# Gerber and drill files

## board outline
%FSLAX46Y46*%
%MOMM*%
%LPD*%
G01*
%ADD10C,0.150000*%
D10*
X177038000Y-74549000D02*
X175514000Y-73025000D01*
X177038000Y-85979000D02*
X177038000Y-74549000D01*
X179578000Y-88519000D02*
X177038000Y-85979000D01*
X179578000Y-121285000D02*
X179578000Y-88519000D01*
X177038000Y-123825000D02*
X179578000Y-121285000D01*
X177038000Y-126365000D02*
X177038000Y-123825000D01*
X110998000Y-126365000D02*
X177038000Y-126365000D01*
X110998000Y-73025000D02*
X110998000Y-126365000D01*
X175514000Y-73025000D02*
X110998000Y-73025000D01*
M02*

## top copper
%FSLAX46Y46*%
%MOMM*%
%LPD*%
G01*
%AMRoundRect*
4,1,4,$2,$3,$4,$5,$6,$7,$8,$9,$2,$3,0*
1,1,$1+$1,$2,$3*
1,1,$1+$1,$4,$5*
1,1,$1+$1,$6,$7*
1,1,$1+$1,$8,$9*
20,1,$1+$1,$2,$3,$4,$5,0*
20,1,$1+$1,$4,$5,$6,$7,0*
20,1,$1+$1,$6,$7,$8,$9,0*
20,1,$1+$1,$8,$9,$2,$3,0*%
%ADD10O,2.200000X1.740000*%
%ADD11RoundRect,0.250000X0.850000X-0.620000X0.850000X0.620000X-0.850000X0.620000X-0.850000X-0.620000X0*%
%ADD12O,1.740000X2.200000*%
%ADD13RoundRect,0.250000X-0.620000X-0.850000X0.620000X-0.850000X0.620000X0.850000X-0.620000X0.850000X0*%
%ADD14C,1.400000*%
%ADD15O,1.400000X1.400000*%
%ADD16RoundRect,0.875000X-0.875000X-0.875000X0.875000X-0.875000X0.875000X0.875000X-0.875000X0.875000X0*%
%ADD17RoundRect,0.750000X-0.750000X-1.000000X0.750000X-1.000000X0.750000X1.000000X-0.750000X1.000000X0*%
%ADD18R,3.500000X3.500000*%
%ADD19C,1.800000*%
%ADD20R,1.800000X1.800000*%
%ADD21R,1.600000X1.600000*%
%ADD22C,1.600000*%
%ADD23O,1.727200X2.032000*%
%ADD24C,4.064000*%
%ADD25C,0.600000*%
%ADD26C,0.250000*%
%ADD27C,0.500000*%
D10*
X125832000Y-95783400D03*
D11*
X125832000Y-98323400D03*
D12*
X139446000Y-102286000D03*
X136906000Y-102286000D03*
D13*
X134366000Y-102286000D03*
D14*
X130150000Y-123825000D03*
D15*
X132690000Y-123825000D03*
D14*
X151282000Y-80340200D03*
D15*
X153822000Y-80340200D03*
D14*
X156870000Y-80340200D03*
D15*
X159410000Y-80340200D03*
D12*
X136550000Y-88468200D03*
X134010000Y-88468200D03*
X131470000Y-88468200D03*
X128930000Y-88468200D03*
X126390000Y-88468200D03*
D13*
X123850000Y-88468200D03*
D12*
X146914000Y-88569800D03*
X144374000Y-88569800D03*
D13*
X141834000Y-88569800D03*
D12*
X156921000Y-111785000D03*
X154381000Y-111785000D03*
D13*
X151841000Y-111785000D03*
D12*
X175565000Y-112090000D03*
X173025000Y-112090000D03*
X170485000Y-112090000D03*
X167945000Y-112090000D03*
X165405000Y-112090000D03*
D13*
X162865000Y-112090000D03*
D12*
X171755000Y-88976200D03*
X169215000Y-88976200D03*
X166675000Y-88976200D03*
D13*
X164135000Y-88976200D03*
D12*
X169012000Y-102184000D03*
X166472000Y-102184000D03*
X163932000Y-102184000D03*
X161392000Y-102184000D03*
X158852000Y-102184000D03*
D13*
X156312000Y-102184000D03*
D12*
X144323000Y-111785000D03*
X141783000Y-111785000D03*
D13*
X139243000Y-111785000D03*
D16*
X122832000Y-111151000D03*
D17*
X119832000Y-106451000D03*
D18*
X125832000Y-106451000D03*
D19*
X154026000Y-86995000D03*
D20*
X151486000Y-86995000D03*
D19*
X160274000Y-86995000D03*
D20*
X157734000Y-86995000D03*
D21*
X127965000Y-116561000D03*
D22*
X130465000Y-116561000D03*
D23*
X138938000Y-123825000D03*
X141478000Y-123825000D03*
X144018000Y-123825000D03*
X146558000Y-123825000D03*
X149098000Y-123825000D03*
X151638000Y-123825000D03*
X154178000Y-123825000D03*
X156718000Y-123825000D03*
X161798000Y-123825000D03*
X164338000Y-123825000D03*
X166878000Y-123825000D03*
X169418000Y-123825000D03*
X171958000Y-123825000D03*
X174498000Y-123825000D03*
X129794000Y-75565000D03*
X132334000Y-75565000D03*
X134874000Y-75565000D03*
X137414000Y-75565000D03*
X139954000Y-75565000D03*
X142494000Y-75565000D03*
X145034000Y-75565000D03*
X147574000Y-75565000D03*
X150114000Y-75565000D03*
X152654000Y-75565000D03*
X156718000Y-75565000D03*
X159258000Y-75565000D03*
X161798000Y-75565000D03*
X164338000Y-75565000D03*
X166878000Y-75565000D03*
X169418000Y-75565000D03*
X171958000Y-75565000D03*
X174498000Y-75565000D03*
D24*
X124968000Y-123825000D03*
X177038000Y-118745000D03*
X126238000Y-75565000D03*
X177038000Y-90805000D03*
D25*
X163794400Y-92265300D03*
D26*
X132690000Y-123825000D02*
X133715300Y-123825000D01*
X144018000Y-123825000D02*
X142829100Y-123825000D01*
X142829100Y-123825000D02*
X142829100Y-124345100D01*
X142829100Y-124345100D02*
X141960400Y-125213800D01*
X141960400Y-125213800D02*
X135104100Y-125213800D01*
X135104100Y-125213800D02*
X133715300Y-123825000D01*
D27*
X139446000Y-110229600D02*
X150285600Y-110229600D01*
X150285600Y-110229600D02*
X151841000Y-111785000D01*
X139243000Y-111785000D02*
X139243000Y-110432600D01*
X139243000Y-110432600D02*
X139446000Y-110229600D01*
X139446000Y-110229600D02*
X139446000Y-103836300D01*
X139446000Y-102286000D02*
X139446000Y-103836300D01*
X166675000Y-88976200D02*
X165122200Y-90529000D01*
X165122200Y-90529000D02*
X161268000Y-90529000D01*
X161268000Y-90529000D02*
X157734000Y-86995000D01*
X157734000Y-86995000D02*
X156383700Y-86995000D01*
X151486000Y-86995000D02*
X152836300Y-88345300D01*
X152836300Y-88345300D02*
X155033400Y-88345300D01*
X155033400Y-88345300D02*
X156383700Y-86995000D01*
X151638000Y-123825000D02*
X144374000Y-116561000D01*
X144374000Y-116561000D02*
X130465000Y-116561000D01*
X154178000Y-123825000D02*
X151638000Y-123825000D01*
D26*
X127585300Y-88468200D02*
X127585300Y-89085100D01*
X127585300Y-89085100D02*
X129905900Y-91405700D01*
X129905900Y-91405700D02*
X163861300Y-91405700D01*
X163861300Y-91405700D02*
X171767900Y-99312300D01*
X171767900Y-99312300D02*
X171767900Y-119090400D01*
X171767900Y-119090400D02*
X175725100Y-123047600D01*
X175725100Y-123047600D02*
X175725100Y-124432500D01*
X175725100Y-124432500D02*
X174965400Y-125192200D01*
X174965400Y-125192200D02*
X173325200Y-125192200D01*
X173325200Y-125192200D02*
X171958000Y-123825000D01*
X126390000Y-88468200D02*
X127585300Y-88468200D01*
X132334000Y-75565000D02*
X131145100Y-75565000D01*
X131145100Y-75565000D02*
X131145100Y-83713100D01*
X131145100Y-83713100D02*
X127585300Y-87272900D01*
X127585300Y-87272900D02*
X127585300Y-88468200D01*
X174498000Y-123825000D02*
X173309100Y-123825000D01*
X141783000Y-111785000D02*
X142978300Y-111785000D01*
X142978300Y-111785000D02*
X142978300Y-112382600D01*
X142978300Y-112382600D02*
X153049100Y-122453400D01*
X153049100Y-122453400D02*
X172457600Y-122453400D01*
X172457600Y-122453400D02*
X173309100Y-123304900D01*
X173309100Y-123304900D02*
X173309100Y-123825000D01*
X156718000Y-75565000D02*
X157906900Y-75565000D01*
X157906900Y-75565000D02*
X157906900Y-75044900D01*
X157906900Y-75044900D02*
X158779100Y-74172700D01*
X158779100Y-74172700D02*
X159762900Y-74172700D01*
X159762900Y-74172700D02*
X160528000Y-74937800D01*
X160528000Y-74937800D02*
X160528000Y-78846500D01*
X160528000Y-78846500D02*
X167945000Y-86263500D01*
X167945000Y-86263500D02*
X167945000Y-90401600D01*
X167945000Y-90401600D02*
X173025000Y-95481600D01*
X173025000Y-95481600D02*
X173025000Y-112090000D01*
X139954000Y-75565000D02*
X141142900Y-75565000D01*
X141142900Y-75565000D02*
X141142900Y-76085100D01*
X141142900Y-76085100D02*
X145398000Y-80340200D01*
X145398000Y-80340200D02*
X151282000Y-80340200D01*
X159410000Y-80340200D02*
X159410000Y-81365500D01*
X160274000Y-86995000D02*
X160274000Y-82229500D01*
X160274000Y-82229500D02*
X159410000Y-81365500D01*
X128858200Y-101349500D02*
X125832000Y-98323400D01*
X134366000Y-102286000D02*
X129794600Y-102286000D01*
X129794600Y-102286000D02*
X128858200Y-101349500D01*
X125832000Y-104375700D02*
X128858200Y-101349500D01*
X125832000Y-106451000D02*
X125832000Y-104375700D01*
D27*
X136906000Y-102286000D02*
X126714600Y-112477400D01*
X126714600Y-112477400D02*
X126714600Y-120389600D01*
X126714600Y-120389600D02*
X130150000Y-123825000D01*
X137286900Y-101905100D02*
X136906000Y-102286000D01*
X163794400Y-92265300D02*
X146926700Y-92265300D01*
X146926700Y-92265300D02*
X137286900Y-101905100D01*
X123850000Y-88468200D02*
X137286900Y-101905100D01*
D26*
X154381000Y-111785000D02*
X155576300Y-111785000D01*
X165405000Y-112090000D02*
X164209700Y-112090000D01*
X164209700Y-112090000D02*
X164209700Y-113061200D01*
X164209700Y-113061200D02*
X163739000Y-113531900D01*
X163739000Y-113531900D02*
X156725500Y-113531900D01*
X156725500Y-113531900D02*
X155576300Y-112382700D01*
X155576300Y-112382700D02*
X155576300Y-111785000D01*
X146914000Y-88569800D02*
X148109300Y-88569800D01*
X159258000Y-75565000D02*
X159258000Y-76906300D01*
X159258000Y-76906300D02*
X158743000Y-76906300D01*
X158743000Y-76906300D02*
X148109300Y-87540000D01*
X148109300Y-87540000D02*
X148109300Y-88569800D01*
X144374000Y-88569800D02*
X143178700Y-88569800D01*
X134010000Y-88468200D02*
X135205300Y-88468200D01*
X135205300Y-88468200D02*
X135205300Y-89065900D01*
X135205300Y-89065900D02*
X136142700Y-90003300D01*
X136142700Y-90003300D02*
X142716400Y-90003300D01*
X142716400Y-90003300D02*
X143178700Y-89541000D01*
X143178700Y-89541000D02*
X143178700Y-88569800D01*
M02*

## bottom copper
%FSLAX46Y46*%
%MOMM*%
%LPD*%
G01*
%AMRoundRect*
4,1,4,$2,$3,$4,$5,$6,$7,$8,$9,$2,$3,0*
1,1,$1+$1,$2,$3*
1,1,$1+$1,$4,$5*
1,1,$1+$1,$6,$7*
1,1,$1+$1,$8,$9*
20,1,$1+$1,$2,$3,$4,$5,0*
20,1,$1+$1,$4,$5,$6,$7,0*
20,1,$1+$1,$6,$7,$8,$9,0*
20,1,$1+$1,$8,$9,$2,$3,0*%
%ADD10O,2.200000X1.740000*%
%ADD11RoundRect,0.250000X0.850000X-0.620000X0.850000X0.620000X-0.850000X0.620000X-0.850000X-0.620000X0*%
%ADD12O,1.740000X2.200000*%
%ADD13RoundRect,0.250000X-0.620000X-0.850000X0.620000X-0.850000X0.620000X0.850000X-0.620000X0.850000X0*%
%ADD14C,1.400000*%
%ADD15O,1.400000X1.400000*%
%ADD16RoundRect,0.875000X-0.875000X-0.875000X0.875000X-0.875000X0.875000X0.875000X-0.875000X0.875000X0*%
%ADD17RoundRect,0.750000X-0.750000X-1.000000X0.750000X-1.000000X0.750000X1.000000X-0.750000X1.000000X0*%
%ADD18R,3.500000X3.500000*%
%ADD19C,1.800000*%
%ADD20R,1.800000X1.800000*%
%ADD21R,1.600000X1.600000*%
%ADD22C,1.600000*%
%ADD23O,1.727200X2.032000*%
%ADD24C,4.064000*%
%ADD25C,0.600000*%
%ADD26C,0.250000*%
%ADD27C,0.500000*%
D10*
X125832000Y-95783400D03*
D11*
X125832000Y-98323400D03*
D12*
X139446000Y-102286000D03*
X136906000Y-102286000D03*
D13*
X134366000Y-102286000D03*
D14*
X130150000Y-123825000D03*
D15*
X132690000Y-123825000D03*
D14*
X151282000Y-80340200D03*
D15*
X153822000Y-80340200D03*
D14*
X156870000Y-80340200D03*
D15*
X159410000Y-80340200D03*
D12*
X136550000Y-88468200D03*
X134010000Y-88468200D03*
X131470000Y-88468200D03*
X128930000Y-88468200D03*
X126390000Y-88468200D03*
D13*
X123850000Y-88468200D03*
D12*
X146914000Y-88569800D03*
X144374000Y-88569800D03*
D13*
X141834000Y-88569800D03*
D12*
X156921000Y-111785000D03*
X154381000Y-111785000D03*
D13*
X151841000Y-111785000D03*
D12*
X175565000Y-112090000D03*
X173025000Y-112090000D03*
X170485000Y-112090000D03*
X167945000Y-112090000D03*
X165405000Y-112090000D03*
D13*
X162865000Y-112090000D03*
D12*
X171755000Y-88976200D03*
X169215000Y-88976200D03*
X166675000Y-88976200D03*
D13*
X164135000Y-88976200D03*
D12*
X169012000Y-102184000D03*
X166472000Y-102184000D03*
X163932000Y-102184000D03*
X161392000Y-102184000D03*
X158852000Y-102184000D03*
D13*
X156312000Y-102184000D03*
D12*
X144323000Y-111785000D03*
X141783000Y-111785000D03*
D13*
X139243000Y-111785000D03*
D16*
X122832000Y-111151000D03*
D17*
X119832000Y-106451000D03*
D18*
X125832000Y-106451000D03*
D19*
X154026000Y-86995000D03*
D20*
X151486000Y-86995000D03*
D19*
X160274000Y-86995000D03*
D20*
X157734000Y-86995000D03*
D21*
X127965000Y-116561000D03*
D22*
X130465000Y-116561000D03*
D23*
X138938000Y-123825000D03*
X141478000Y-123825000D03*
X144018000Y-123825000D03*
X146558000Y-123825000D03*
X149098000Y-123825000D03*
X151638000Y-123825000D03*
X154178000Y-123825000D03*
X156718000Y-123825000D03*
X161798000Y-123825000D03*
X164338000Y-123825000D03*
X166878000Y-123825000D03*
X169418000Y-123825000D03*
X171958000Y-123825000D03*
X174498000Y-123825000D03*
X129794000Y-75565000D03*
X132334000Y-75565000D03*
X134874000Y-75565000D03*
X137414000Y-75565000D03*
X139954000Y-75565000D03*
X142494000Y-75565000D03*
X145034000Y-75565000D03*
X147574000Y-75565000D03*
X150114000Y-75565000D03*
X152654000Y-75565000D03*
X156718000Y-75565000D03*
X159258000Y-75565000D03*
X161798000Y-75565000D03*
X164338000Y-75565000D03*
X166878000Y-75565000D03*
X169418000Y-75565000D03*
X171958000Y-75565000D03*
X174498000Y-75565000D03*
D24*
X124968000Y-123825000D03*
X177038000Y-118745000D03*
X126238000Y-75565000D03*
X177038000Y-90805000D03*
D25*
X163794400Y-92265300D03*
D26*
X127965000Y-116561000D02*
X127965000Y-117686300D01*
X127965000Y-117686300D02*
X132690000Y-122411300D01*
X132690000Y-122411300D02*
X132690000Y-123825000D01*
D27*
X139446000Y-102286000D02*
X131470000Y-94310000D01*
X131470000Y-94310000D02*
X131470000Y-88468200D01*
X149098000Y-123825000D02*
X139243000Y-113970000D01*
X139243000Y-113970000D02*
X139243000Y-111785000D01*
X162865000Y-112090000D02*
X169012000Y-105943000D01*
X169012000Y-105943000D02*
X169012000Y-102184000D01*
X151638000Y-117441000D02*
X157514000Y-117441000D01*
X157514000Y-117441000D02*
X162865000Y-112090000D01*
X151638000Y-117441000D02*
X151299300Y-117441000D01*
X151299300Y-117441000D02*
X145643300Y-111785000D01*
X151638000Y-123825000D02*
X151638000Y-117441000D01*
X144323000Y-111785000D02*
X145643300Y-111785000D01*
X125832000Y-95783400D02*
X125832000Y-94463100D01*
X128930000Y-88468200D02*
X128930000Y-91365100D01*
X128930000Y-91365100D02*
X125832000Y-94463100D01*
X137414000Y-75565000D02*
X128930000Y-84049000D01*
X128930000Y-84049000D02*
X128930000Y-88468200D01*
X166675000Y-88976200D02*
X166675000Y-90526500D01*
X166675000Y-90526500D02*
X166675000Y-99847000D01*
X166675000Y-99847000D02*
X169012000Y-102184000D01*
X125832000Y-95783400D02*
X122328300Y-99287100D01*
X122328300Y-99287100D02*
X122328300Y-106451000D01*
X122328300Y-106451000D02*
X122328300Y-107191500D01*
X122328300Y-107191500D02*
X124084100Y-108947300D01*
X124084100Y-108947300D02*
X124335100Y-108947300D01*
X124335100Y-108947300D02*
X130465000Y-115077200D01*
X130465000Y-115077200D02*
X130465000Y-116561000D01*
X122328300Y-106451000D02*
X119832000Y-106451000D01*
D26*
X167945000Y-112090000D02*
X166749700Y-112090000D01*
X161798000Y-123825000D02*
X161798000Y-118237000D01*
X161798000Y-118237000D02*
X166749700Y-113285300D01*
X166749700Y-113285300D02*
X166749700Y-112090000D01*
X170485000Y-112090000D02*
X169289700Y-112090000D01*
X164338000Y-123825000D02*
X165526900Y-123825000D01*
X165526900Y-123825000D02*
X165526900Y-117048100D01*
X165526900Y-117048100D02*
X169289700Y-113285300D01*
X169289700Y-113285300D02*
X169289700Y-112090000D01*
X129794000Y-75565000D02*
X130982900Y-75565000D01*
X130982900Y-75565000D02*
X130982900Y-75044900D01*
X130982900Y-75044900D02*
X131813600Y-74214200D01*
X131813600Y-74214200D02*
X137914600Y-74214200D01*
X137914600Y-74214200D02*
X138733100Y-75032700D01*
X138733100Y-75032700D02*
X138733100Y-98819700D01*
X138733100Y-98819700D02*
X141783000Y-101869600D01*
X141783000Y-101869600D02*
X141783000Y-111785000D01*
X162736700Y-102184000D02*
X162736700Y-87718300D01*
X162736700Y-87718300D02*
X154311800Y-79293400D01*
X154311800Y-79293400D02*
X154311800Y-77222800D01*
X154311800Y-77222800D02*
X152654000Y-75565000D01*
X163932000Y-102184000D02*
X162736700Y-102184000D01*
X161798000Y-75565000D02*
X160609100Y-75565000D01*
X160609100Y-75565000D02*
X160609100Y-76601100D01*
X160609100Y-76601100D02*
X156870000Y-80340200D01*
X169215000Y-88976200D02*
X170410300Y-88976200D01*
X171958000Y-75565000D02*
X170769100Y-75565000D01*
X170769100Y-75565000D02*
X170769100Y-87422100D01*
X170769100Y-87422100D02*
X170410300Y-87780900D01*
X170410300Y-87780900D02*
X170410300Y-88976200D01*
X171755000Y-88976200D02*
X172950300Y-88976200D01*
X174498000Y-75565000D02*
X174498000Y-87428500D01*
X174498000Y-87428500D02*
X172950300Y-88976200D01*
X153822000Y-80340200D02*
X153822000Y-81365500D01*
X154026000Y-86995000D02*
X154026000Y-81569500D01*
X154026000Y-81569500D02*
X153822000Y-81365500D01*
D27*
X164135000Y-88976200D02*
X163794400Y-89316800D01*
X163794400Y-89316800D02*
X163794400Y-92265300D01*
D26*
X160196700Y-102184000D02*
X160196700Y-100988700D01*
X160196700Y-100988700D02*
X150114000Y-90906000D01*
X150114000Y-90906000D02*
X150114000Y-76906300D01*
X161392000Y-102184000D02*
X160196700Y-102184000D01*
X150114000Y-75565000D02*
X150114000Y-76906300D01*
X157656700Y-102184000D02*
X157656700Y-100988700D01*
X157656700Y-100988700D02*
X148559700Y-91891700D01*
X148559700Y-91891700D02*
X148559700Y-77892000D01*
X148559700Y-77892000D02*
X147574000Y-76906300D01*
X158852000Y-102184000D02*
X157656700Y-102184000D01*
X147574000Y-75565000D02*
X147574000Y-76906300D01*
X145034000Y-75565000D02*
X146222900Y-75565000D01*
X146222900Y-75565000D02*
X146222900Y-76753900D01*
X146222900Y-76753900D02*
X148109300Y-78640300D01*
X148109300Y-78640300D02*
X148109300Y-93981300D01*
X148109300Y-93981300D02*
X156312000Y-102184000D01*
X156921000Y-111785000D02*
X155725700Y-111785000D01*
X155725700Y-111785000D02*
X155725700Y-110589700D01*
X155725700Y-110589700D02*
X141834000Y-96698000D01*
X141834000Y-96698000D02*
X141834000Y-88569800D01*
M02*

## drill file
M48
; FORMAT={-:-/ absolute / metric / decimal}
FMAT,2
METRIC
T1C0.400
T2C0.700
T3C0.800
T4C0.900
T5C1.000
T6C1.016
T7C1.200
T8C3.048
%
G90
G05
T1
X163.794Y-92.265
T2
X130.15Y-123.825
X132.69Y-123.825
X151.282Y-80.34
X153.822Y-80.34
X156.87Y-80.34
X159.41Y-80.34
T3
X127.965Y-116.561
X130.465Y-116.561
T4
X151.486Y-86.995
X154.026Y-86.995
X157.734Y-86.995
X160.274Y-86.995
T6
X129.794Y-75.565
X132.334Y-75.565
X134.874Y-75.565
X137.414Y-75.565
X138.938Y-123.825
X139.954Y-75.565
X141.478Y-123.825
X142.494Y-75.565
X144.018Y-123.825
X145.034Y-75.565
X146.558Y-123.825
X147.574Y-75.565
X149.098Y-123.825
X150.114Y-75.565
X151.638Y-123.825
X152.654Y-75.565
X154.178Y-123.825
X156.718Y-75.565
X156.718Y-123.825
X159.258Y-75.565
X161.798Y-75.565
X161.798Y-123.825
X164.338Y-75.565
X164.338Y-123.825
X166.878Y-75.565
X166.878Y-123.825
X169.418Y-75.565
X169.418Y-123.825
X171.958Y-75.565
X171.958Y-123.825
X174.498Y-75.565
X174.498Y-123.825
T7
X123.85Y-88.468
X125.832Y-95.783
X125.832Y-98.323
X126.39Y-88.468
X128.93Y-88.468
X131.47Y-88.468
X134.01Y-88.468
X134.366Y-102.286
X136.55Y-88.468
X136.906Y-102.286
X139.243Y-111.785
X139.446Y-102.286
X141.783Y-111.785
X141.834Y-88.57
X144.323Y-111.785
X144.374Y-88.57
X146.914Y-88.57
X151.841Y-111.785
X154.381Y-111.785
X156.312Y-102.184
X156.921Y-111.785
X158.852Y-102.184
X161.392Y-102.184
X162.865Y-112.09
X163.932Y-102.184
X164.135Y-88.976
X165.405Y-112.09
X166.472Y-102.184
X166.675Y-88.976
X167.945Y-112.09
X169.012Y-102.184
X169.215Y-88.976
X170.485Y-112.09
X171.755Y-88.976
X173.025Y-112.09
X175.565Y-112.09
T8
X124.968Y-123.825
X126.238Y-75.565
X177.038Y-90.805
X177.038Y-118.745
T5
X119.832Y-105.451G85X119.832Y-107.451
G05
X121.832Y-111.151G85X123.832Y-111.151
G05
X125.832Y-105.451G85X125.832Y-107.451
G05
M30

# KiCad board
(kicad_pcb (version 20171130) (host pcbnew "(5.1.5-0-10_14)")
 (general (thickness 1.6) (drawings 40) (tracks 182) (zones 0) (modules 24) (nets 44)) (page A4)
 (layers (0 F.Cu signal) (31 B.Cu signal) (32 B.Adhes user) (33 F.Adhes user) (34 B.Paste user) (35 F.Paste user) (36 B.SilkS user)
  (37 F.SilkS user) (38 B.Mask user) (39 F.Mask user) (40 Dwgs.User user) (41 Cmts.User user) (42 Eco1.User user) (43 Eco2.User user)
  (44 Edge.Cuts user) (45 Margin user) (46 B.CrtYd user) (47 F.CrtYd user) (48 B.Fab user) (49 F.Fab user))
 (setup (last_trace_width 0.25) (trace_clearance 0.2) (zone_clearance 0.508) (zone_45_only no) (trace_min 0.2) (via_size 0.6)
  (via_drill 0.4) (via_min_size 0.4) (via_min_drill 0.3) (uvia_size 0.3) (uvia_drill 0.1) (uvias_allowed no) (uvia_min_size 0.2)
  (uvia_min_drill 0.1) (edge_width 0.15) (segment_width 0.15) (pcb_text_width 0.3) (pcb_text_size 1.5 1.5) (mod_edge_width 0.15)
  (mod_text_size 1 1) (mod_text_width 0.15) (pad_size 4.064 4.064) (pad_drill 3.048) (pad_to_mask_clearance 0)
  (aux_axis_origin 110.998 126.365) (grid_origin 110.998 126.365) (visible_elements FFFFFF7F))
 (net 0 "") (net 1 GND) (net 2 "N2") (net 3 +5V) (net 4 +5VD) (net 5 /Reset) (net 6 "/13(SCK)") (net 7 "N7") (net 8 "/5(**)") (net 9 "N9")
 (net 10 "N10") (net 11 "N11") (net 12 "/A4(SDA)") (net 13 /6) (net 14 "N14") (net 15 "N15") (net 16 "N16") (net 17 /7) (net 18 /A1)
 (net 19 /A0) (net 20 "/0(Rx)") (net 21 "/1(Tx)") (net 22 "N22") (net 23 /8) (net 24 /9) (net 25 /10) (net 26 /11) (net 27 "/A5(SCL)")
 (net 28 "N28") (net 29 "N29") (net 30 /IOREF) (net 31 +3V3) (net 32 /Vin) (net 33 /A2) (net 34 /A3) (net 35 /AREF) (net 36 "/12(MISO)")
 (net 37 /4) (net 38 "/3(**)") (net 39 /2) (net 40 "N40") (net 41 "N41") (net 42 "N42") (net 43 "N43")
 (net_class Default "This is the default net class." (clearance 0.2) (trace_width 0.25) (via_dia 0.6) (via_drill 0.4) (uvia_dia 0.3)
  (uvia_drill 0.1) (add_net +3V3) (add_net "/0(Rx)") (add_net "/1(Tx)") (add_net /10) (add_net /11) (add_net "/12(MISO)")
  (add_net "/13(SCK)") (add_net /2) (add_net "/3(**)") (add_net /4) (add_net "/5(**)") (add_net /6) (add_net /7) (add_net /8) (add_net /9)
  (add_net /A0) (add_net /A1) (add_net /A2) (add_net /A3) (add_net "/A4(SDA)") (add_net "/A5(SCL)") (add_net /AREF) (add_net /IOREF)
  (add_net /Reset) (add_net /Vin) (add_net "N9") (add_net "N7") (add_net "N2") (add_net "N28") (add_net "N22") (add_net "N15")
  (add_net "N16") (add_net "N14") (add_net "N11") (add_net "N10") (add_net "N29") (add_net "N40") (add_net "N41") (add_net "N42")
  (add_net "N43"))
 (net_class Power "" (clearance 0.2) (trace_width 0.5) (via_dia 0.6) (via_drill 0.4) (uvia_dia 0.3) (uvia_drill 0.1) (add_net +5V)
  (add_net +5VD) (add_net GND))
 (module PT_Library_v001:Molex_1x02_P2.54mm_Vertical (layer F.Cu) (at 125.832 98.3234 90)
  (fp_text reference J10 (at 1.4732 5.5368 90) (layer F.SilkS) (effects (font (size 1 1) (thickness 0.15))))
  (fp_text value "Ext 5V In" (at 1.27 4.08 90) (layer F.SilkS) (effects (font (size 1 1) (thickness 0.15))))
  (pad 2 thru_hole oval (at 2.54 0 90) (size 1.74 2.2) (drill 1.2) (layers *.Cu *.Mask) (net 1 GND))
  (pad 1 thru_hole roundrect (at 0 0 90) (size 1.74 2.2) (drill 1.2) (layers *.Cu *.Mask) (roundrect_rratio 0.143678) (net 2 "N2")))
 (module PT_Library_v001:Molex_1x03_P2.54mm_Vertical (layer F.Cu) (at 134.366 102.286)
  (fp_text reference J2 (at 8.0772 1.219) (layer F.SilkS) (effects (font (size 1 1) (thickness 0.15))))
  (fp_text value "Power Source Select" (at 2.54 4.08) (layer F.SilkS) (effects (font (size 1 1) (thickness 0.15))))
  (pad 3 thru_hole oval (at 5.08 0) (size 1.74 2.2) (drill 1.2) (layers *.Cu *.Mask) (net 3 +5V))
  (pad 2 thru_hole oval (at 2.54 0) (size 1.74 2.2) (drill 1.2) (layers *.Cu *.Mask) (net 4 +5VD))
  (pad 1 thru_hole roundrect (at 0 0) (size 1.74 2.2) (drill 1.2) (layers *.Cu *.Mask) (roundrect_rratio 0.143678) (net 2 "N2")))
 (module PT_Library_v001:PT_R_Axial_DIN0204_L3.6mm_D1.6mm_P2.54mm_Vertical (layer F.Cu) (at 130.15 123.825)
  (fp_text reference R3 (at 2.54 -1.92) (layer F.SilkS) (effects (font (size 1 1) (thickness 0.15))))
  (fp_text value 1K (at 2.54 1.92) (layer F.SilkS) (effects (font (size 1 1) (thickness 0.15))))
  (pad 1 thru_hole circle (at 0 0) (size 1.4 1.4) (drill 0.7) (layers *.Cu *.Mask) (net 4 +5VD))
  (pad 2 thru_hole oval (at 2.54 0) (size 1.4 1.4) (drill 0.7) (layers *.Cu *.Mask) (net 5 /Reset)))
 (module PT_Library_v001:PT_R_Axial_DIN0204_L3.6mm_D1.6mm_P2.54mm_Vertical (layer F.Cu) (at 151.282 80.3402)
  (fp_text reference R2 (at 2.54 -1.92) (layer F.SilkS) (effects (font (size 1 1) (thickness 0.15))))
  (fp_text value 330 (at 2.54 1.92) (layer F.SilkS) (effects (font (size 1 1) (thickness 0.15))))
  (pad 1 thru_hole circle (at 0 0) (size 1.4 1.4) (drill 0.7) (layers *.Cu *.Mask) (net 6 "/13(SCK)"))
  (pad 2 thru_hole oval (at 2.54 0) (size 1.4 1.4) (drill 0.7) (layers *.Cu *.Mask) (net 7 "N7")))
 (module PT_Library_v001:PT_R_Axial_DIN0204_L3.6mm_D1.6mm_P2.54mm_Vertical (layer F.Cu) (at 156.87 80.3402)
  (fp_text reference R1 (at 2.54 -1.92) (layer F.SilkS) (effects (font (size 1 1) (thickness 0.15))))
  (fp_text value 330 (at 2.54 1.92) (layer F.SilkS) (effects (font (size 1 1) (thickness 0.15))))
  (pad 1 thru_hole circle (at 0 0) (size 1.4 1.4) (drill 0.7) (layers *.Cu *.Mask) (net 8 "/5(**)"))
  (pad 2 thru_hole oval (at 2.54 0) (size 1.4 1.4) (drill 0.7) (layers *.Cu *.Mask) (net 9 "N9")))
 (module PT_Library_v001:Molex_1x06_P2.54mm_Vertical (layer F.Cu) (at 123.85 88.4682)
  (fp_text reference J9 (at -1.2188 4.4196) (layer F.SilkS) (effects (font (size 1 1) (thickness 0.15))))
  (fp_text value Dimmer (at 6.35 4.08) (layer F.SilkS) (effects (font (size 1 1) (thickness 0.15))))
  (pad 6 thru_hole oval (at 12.7 0) (size 1.74 2.2) (drill 1.2) (layers *.Cu *.Mask) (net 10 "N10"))
  (pad 5 thru_hole oval (at 10.16 0) (size 1.74 2.2) (drill 1.2) (layers *.Cu *.Mask) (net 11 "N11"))
  (pad 4 thru_hole oval (at 7.62 0) (size 1.74 2.2) (drill 1.2) (layers *.Cu *.Mask) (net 3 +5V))
  (pad 3 thru_hole oval (at 5.08 0) (size 1.74 2.2) (drill 1.2) (layers *.Cu *.Mask) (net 1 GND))
  (pad 2 thru_hole oval (at 2.54 0) (size 1.74 2.2) (drill 1.2) (layers *.Cu *.Mask) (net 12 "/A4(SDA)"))
  (pad 1 thru_hole roundrect (at 0 0) (size 1.74 2.2) (drill 1.2) (layers *.Cu *.Mask) (roundrect_rratio 0.143678) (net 4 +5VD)))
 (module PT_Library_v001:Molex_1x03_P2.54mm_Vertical (layer F.Cu) (at 141.834 88.5698)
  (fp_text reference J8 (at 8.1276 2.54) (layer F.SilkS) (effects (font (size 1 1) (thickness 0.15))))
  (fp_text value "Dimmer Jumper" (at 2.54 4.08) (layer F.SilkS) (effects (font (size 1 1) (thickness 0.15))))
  (pad 3 thru_hole oval (at 5.08 0) (size 1.74 2.2) (drill 1.2) (layers *.Cu *.Mask) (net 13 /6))
  (pad 2 thru_hole oval (at 2.54 0) (size 1.74 2.2) (drill 1.2) (layers *.Cu *.Mask) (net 11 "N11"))
  (pad 1 thru_hole roundrect (at 0 0) (size 1.74 2.2) (drill 1.2) (layers *.Cu *.Mask) (roundrect_rratio 0.143678) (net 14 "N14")))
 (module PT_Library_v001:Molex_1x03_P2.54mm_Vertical (layer F.Cu) (at 151.841 111.785)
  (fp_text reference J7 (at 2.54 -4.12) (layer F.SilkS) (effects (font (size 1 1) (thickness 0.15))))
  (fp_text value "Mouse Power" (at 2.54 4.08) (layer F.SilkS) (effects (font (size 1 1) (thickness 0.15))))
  (pad 3 thru_hole oval (at 5.08 0) (size 1.74 2.2) (drill 1.2) (layers *.Cu *.Mask) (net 14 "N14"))
  (pad 2 thru_hole oval (at 2.54 0) (size 1.74 2.2) (drill 1.2) (layers *.Cu *.Mask) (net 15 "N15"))
  (pad 1 thru_hole roundrect (at 0 0) (size 1.74 2.2) (drill 1.2) (layers *.Cu *.Mask) (roundrect_rratio 0.143678) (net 3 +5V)))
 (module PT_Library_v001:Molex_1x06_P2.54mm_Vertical (layer F.Cu) (at 162.865 112.09)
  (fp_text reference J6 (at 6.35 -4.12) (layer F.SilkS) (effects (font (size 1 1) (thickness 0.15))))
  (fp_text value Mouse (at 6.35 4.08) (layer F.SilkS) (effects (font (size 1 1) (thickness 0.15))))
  (pad 6 thru_hole oval (at 12.7 0) (size 1.74 2.2) (drill 1.2) (layers *.Cu *.Mask) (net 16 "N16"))
  (pad 5 thru_hole oval (at 10.16 0) (size 1.74 2.2) (drill 1.2) (layers *.Cu *.Mask) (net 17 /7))
  (pad 4 thru_hole oval (at 7.62 0) (size 1.74 2.2) (drill 1.2) (layers *.Cu *.Mask) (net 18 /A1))
  (pad 3 thru_hole oval (at 5.08 0) (size 1.74 2.2) (drill 1.2) (layers *.Cu *.Mask) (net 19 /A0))
  (pad 2 thru_hole oval (at 2.54 0) (size 1.74 2.2) (drill 1.2) (layers *.Cu *.Mask) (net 15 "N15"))
  (pad 1 thru_hole roundrect (at 0 0) (size 1.74 2.2) (drill 1.2) (layers *.Cu *.Mask) (roundrect_rratio 0.143678) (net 1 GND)))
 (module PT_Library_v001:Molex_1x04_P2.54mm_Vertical (layer F.Cu) (at 164.135 88.9762)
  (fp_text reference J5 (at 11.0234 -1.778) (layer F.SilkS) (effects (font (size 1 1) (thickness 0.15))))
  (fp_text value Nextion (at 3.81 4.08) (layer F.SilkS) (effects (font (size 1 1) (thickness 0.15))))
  (pad 4 thru_hole oval (at 7.62 0) (size 1.74 2.2) (drill 1.2) (layers *.Cu *.Mask) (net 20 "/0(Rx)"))
  (pad 3 thru_hole oval (at 5.08 0) (size 1.74 2.2) (drill 1.2) (layers *.Cu *.Mask) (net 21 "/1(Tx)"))
  (pad 2 thru_hole oval (at 2.54 0) (size 1.74 2.2) (drill 1.2) (layers *.Cu *.Mask) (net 1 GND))
  (pad 1 thru_hole roundrect (at 0 0) (size 1.74 2.2) (drill 1.2) (layers *.Cu *.Mask) (roundrect_rratio 0.143678) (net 4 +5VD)))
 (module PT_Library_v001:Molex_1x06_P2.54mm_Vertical (layer F.Cu) (at 156.312 102.184)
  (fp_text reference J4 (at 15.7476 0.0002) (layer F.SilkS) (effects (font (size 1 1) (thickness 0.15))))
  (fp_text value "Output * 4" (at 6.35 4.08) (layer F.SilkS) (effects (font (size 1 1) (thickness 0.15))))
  (pad 6 thru_hole oval (at 12.7 0) (size 1.74 2.2) (drill 1.2) (layers *.Cu *.Mask) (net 1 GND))
  (pad 5 thru_hole oval (at 10.16 0) (size 1.74 2.2) (drill 1.2) (layers *.Cu *.Mask) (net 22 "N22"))
  (pad 4 thru_hole oval (at 7.62 0) (size 1.74 2.2) (drill 1.2) (layers *.Cu *.Mask) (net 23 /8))
  (pad 3 thru_hole oval (at 5.08 0) (size 1.74 2.2) (drill 1.2) (layers *.Cu *.Mask) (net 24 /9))
  (pad 2 thru_hole oval (at 2.54 0) (size 1.74 2.2) (drill 1.2) (layers *.Cu *.Mask) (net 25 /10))
  (pad 1 thru_hole roundrect (at 0 0) (size 1.74 2.2) (drill 1.2) (layers *.Cu *.Mask) (roundrect_rratio 0.143678) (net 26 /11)))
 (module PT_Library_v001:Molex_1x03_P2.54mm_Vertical (layer F.Cu) (at 139.243 111.785)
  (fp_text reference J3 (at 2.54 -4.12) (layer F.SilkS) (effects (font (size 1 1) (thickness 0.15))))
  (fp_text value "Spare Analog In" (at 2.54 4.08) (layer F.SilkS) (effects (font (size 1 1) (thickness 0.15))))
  (pad 3 thru_hole oval (at 5.08 0) (size 1.74 2.2) (drill 1.2) (layers *.Cu *.Mask) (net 1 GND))
  (pad 2 thru_hole oval (at 2.54 0) (size 1.74 2.2) (drill 1.2) (layers *.Cu *.Mask) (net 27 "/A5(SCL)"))
  (pad 1 thru_hole roundrect (at 0 0) (size 1.74 2.2) (drill 1.2) (layers *.Cu *.Mask) (roundrect_rratio 0.143678) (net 3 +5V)))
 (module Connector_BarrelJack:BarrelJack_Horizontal (layer F.Cu) (at 125.832 106.451)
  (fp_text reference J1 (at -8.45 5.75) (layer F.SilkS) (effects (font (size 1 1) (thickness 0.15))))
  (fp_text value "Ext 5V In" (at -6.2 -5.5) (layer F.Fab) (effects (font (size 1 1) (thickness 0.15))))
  (pad 3 thru_hole roundrect (at -3 4.7) (size 3.5 3.5) (drill oval 3 1) (layers *.Cu *.Mask) (roundrect_rratio 0.25) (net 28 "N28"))
  (pad 2 thru_hole roundrect (at -6 0) (size 3 3.5) (drill oval 1 3) (layers *.Cu *.Mask) (roundrect_rratio 0.25) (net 1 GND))
  (pad 1 thru_hole rect (at 0 0) (size 3.5 3.5) (drill oval 1 3) (layers *.Cu *.Mask) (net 2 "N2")))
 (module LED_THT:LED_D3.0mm (layer F.Cu) (at 151.486 86.995)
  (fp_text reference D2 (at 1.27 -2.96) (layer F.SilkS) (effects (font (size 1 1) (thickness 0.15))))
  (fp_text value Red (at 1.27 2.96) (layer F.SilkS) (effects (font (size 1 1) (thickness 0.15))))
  (pad 2 thru_hole circle (at 2.54 0) (size 1.8 1.8) (drill 0.9) (layers *.Cu *.Mask) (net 7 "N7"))
  (pad 1 thru_hole rect (at 0 0) (size 1.8 1.8) (drill 0.9) (layers *.Cu *.Mask) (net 1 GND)))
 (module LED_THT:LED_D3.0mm (layer F.Cu) (at 157.734 86.995)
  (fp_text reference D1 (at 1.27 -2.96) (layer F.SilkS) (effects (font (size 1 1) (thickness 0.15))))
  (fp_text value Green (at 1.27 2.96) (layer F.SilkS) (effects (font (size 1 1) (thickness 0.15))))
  (pad 2 thru_hole circle (at 2.54 0) (size 1.8 1.8) (drill 0.9) (layers *.Cu *.Mask) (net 9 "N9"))
  (pad 1 thru_hole rect (at 0 0) (size 1.8 1.8) (drill 0.9) (layers *.Cu *.Mask) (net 1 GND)))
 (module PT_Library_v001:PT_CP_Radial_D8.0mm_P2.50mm (layer F.Cu) (at 127.965 116.561)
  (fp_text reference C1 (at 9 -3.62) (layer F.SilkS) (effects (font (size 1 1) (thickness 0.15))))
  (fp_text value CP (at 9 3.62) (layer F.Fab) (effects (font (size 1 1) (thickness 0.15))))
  (pad 1 thru_hole rect (at 0 0) (size 1.6 1.6) (drill 0.8) (layers *.Cu *.Mask) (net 5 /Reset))
  (pad 2 thru_hole circle (at 2.5 0) (size 1.6 1.6) (drill 0.8) (layers *.Cu *.Mask) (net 1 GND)))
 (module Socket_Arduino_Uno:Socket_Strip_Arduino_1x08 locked (layer F.Cu) (at 138.938 123.825)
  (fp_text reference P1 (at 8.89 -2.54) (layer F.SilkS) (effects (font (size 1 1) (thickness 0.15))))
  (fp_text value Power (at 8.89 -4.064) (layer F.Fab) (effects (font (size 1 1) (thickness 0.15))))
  (pad 1 thru_hole oval (at 0 0) (size 1.7272 2.032) (drill 1.016) (layers *.Cu *.Mask F.SilkS) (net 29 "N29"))
  (pad 2 thru_hole oval (at 2.54 0) (size 1.7272 2.032) (drill 1.016) (layers *.Cu *.Mask F.SilkS) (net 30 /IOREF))
  (pad 3 thru_hole oval (at 5.08 0) (size 1.7272 2.032) (drill 1.016) (layers *.Cu *.Mask F.SilkS) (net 5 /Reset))
  (pad 4 thru_hole oval (at 7.62 0) (size 1.7272 2.032) (drill 1.016) (layers *.Cu *.Mask F.SilkS) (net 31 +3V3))
  (pad 5 thru_hole oval (at 10.16 0) (size 1.7272 2.032) (drill 1.016) (layers *.Cu *.Mask F.SilkS) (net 3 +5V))
  (pad 6 thru_hole oval (at 12.7 0) (size 1.7272 2.032) (drill 1.016) (layers *.Cu *.Mask F.SilkS) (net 1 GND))
  (pad 7 thru_hole oval (at 15.24 0) (size 1.7272 2.032) (drill 1.016) (layers *.Cu *.Mask F.SilkS) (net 1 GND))
  (pad 8 thru_hole oval (at 17.78 0) (size 1.7272 2.032) (drill 1.016) (layers *.Cu *.Mask F.SilkS) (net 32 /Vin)))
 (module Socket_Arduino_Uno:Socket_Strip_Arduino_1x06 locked (layer F.Cu) (at 161.798 123.825)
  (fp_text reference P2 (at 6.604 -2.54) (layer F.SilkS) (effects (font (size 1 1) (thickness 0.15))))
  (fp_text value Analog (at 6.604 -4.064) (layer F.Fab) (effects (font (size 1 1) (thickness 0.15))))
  (pad 1 thru_hole oval (at 0 0) (size 1.7272 2.032) (drill 1.016) (layers *.Cu *.Mask F.SilkS) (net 19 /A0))
  (pad 2 thru_hole oval (at 2.54 0) (size 1.7272 2.032) (drill 1.016) (layers *.Cu *.Mask F.SilkS) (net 18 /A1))
  (pad 3 thru_hole oval (at 5.08 0) (size 1.7272 2.032) (drill 1.016) (layers *.Cu *.Mask F.SilkS) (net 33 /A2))
  (pad 4 thru_hole oval (at 7.62 0) (size 1.7272 2.032) (drill 1.016) (layers *.Cu *.Mask F.SilkS) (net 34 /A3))
  (pad 5 thru_hole oval (at 10.16 0) (size 1.7272 2.032) (drill 1.016) (layers *.Cu *.Mask F.SilkS) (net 12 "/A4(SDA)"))
  (pad 6 thru_hole oval (at 12.7 0) (size 1.7272 2.032) (drill 1.016) (layers *.Cu *.Mask F.SilkS) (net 27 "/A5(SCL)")))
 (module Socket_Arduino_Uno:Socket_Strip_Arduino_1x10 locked (layer F.Cu) (at 129.794 75.565)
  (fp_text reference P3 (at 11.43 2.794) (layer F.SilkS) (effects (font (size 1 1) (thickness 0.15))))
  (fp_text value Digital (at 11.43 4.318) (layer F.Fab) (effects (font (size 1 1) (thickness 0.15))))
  (pad 1 thru_hole oval (at 0 0) (size 1.7272 2.032) (drill 1.016) (layers *.Cu *.Mask F.SilkS) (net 27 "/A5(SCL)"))
  (pad 2 thru_hole oval (at 2.54 0) (size 1.7272 2.032) (drill 1.016) (layers *.Cu *.Mask F.SilkS) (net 12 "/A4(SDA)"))
  (pad 3 thru_hole oval (at 5.08 0) (size 1.7272 2.032) (drill 1.016) (layers *.Cu *.Mask F.SilkS) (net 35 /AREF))
  (pad 4 thru_hole oval (at 7.62 0) (size 1.7272 2.032) (drill 1.016) (layers *.Cu *.Mask F.SilkS) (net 1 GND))
  (pad 5 thru_hole oval (at 10.16 0) (size 1.7272 2.032) (drill 1.016) (layers *.Cu *.Mask F.SilkS) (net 6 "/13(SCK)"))
  (pad 6 thru_hole oval (at 12.7 0) (size 1.7272 2.032) (drill 1.016) (layers *.Cu *.Mask F.SilkS) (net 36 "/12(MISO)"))
  (pad 7 thru_hole oval (at 15.24 0) (size 1.7272 2.032) (drill 1.016) (layers *.Cu *.Mask F.SilkS) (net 26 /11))
  (pad 8 thru_hole oval (at 17.78 0) (size 1.7272 2.032) (drill 1.016) (layers *.Cu *.Mask F.SilkS) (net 25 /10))
  (pad 9 thru_hole oval (at 20.32 0) (size 1.7272 2.032) (drill 1.016) (layers *.Cu *.Mask F.SilkS) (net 24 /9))
  (pad 10 thru_hole oval (at 22.86 0) (size 1.7272 2.032) (drill 1.016) (layers *.Cu *.Mask F.SilkS) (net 23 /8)))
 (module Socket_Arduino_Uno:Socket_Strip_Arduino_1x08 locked (layer F.Cu) (at 156.718 75.565)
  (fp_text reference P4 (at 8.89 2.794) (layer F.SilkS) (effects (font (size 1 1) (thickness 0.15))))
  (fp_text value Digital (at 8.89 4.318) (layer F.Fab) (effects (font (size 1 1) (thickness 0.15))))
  (pad 1 thru_hole oval (at 0 0) (size 1.7272 2.032) (drill 1.016) (layers *.Cu *.Mask F.SilkS) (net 17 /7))
  (pad 2 thru_hole oval (at 2.54 0) (size 1.7272 2.032) (drill 1.016) (layers *.Cu *.Mask F.SilkS) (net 13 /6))
  (pad 3 thru_hole oval (at 5.08 0) (size 1.7272 2.032) (drill 1.016) (layers *.Cu *.Mask F.SilkS) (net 8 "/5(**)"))
  (pad 4 thru_hole oval (at 7.62 0) (size 1.7272 2.032) (drill 1.016) (layers *.Cu *.Mask F.SilkS) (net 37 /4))
  (pad 5 thru_hole oval (at 10.16 0) (size 1.7272 2.032) (drill 1.016) (layers *.Cu *.Mask F.SilkS) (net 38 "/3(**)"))
  (pad 6 thru_hole oval (at 12.7 0) (size 1.7272 2.032) (drill 1.016) (layers *.Cu *.Mask F.SilkS) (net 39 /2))
  (pad 7 thru_hole oval (at 15.24 0) (size 1.7272 2.032) (drill 1.016) (layers *.Cu *.Mask F.SilkS) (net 21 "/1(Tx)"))
  (pad 8 thru_hole oval (at 17.78 0) (size 1.7272 2.032) (drill 1.016) (layers *.Cu *.Mask F.SilkS) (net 20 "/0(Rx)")))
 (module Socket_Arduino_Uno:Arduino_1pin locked (layer F.Cu) (at 124.968 123.825)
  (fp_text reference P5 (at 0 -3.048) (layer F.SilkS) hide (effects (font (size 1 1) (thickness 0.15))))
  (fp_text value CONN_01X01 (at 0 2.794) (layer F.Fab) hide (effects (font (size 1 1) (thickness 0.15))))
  (pad 1 thru_hole circle (at 0 0) (size 4.064 4.064) (drill 3.048) (layers *.Cu *.Mask F.SilkS) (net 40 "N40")))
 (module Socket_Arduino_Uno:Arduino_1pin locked (layer F.Cu) (at 177.038 118.745)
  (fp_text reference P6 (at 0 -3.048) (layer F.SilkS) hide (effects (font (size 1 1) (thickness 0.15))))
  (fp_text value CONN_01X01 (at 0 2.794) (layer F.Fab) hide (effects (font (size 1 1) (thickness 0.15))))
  (pad 1 thru_hole circle (at 0 0) (size 4.064 4.064) (drill 3.048) (layers *.Cu *.Mask F.SilkS) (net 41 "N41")))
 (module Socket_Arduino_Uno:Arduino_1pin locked (layer F.Cu) (at 126.238 75.565)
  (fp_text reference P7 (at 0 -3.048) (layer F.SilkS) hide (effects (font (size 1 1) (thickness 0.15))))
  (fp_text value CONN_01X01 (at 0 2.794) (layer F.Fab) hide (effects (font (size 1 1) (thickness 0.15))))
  (pad 1 thru_hole circle (at 0 0) (size 4.064 4.064) (drill 3.048) (layers *.Cu *.Mask F.SilkS) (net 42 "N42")))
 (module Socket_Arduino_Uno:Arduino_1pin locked (layer F.Cu) (at 177.038 90.805)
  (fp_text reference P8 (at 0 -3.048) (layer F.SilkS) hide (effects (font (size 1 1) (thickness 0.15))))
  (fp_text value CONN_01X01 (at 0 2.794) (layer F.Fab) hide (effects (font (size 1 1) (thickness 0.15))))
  (pad 1 thru_hole circle (at 0 0) (size 4.064 4.064) (drill 3.048) (layers *.Cu *.Mask F.SilkS) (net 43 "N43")))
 (gr_line (start 177.038 74.549) (end 175.514 73.025) (angle 90) (layer Edge.Cuts) (width 0.15))
 (gr_line (start 177.038 85.979) (end 177.038 74.549) (angle 90) (layer Edge.Cuts) (width 0.15))
 (gr_line (start 179.578 88.519) (end 177.038 85.979) (angle 90) (layer Edge.Cuts) (width 0.15))
 (gr_line (start 179.578 121.285) (end 179.578 88.519) (angle 90) (layer Edge.Cuts) (width 0.15))
 (gr_line (start 177.038 123.825) (end 179.578 121.285) (angle 90) (layer Edge.Cuts) (width 0.15))
 (gr_line (start 177.038 126.365) (end 177.038 123.825) (angle 90) (layer Edge.Cuts) (width 0.15))
 (gr_line (start 110.998 126.365) (end 177.038 126.365) (angle 90) (layer Edge.Cuts) (width 0.15))
 (gr_line (start 110.998 73.025) (end 110.998 126.365) (angle 90) (layer Edge.Cuts) (width 0.15))
 (gr_line (start 175.514 73.025) (end 110.998 73.025) (angle 90) (layer Edge.Cuts) (width 0.15))
 (segment (start 127.965 116.561) (end 127.965 117.6863) (width 0.25) (layer B.Cu) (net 5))
 (segment (start 127.965 117.6863) (end 132.69 122.4113) (width 0.25) (layer B.Cu) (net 5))
 (segment (start 132.69 122.4113) (end 132.69 123.825) (width 0.25) (layer B.Cu) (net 5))
 (segment (start 132.69 123.825) (end 133.7153 123.825) (width 0.25) (layer F.Cu) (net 5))
 (segment (start 144.018 123.825) (end 142.8291 123.825) (width 0.25) (layer F.Cu) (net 5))
 (segment (start 142.8291 123.825) (end 142.8291 124.3451) (width 0.25) (layer F.Cu) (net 5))
 (segment (start 142.8291 124.3451) (end 141.9604 125.2138) (width 0.25) (layer F.Cu) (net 5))
 (segment (start 141.9604 125.2138) (end 135.1041 125.2138) (width 0.25) (layer F.Cu) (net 5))
 (segment (start 135.1041 125.2138) (end 133.7153 123.825) (width 0.25) (layer F.Cu) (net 5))
 (segment (start 139.446 102.286) (end 131.47 94.31) (width 0.5) (layer B.Cu) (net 3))
 (segment (start 131.47 94.31) (end 131.47 88.4682) (width 0.5) (layer B.Cu) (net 3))
 (segment (start 139.446 110.2296) (end 150.2856 110.2296) (width 0.5) (layer F.Cu) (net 3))
 (segment (start 150.2856 110.2296) (end 151.841 111.785) (width 0.5) (layer F.Cu) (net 3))
 (segment (start 139.243 111.785) (end 139.243 110.4326) (width 0.5) (layer F.Cu) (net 3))
 (segment (start 139.243 110.4326) (end 139.446 110.2296) (width 0.5) (layer F.Cu) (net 3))
 (segment (start 139.446 110.2296) (end 139.446 103.8363) (width 0.5) (layer F.Cu) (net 3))
 (segment (start 139.446 102.286) (end 139.446 103.8363) (width 0.5) (layer F.Cu) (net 3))
 (segment (start 149.098 123.825) (end 139.243 113.97) (width 0.5) (layer B.Cu) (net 3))
 (segment (start 139.243 113.97) (end 139.243 111.785) (width 0.5) (layer B.Cu) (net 3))
 (segment (start 162.865 112.09) (end 169.012 105.943) (width 0.5) (layer B.Cu) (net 1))
 (segment (start 169.012 105.943) (end 169.012 102.184) (width 0.5) (layer B.Cu) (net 1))
 (segment (start 151.638 117.441) (end 157.514 117.441) (width 0.5) (layer B.Cu) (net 1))
 (segment (start 157.514 117.441) (end 162.865 112.09) (width 0.5) (layer B.Cu) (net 1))
 (segment (start 151.638 117.441) (end 151.2993 117.441) (width 0.5) (layer B.Cu) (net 1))
 (segment (start 151.2993 117.441) (end 145.6433 111.785) (width 0.5) (layer B.Cu) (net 1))
 (segment (start 151.638 123.825) (end 151.638 117.441) (width 0.5) (layer B.Cu) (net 1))
 (segment (start 144.323 111.785) (end 145.6433 111.785) (width 0.5) (layer B.Cu) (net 1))
 (segment (start 125.832 95.7834) (end 125.832 94.4631) (width 0.5) (layer B.Cu) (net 1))
 (segment (start 128.93 88.4682) (end 128.93 91.3651) (width 0.5) (layer B.Cu) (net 1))
 (segment (start 128.93 91.3651) (end 125.832 94.4631) (width 0.5) (layer B.Cu) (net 1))
 (segment (start 137.414 75.565) (end 128.93 84.049) (width 0.5) (layer B.Cu) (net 1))
 (segment (start 128.93 84.049) (end 128.93 88.4682) (width 0.5) (layer B.Cu) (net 1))
 (segment (start 166.675 88.9762) (end 166.675 90.5265) (width 0.5) (layer B.Cu) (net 1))
 (segment (start 166.675 90.5265) (end 166.675 99.847) (width 0.5) (layer B.Cu) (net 1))
 (segment (start 166.675 99.847) (end 169.012 102.184) (width 0.5) (layer B.Cu) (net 1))
 (segment (start 166.675 88.9762) (end 165.1222 90.529) (width 0.5) (layer F.Cu) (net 1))
 (segment (start 165.1222 90.529) (end 161.268 90.529) (width 0.5) (layer F.Cu) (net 1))
 (segment (start 161.268 90.529) (end 157.734 86.995) (width 0.5) (layer F.Cu) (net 1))
 (segment (start 157.734 86.995) (end 156.3837 86.995) (width 0.5) (layer F.Cu) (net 1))
 (segment (start 151.486 86.995) (end 152.8363 88.3453) (width 0.5) (layer F.Cu) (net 1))
 (segment (start 152.8363 88.3453) (end 155.0334 88.3453) (width 0.5) (layer F.Cu) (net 1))
 (segment (start 155.0334 88.3453) (end 156.3837 86.995) (width 0.5) (layer F.Cu) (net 1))
 (segment (start 125.832 95.7834) (end 122.3283 99.2871) (width 0.5) (layer B.Cu) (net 1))
 (segment (start 122.3283 99.2871) (end 122.3283 106.451) (width 0.5) (layer B.Cu) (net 1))
 (segment (start 122.3283 106.451) (end 122.3283 107.1915) (width 0.5) (layer B.Cu) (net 1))
 (segment (start 122.3283 107.1915) (end 124.0841 108.9473) (width 0.5) (layer B.Cu) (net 1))
 (segment (start 124.0841 108.9473) (end 124.3351 108.9473) (width 0.5) (layer B.Cu) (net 1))
 (segment (start 124.3351 108.9473) (end 130.465 115.0772) (width 0.5) (layer B.Cu) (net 1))
 (segment (start 130.465 115.0772) (end 130.465 116.561) (width 0.5) (layer B.Cu) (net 1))
 (segment (start 122.3283 106.451) (end 119.832 106.451) (width 0.5) (layer B.Cu) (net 1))
 (segment (start 151.638 123.825) (end 144.374 116.561) (width 0.5) (layer F.Cu) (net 1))
 (segment (start 144.374 116.561) (end 130.465 116.561) (width 0.5) (layer F.Cu) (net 1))
 (segment (start 154.178 123.825) (end 151.638 123.825) (width 0.5) (layer F.Cu) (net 1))
 (segment (start 167.945 112.09) (end 166.7497 112.09) (width 0.25) (layer B.Cu) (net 19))
 (segment (start 161.798 123.825) (end 161.798 118.237) (width 0.25) (layer B.Cu) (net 19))
 (segment (start 161.798 118.237) (end 166.7497 113.2853) (width 0.25) (layer B.Cu) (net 19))
 (segment (start 166.7497 113.2853) (end 166.7497 112.09) (width 0.25) (layer B.Cu) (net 19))
 (segment (start 170.485 112.09) (end 169.2897 112.09) (width 0.25) (layer B.Cu) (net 18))
 (segment (start 164.338 123.825) (end 165.5269 123.825) (width 0.25) (layer B.Cu) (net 18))
 (segment (start 165.5269 123.825) (end 165.5269 117.0481) (width 0.25) (layer B.Cu) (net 18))
 (segment (start 165.5269 117.0481) (end 169.2897 113.2853) (width 0.25) (layer B.Cu) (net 18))
 (segment (start 169.2897 113.2853) (end 169.2897 112.09) (width 0.25) (layer B.Cu) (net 18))
 (segment (start 127.5853 88.4682) (end 127.5853 89.0851) (width 0.25) (layer F.Cu) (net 12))
 (segment (start 127.5853 89.0851) (end 129.9059 91.4057) (width 0.25) (layer F.Cu) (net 12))
 (segment (start 129.9059 91.4057) (end 163.8613 91.4057) (width 0.25) (layer F.Cu) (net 12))
 (segment (start 163.8613 91.4057) (end 171.7679 99.3123) (width 0.25) (layer F.Cu) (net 12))
 (segment (start 171.7679 99.3123) (end 171.7679 119.0904) (width 0.25) (layer F.Cu) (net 12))
 (segment (start 171.7679 119.0904) (end 175.7251 123.0476) (width 0.25) (layer F.Cu) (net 12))
 (segment (start 175.7251 123.0476) (end 175.7251 124.4325) (width 0.25) (layer F.Cu) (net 12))
 (segment (start 175.7251 124.4325) (end 174.9654 125.1922) (width 0.25) (layer F.Cu) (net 12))
 (segment (start 174.9654 125.1922) (end 173.3252 125.1922) (width 0.25) (layer F.Cu) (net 12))
 (segment (start 173.3252 125.1922) (end 171.958 123.825) (width 0.25) (layer F.Cu) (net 12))
 (segment (start 126.39 88.4682) (end 127.5853 88.4682) (width 0.25) (layer F.Cu) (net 12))
 (segment (start 132.334 75.565) (end 131.1451 75.565) (width 0.25) (layer F.Cu) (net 12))
 (segment (start 131.1451 75.565) (end 131.1451 83.7131) (width 0.25) (layer F.Cu) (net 12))
 (segment (start 131.1451 83.7131) (end 127.5853 87.2729) (width 0.25) (layer F.Cu) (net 12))
 (segment (start 127.5853 87.2729) (end 127.5853 88.4682) (width 0.25) (layer F.Cu) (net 12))
 (segment (start 129.794 75.565) (end 130.9829 75.565) (width 0.25) (layer B.Cu) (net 27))
 (segment (start 174.498 123.825) (end 173.3091 123.825) (width 0.25) (layer F.Cu) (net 27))
 (segment (start 141.783 111.785) (end 142.9783 111.785) (width 0.25) (layer F.Cu) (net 27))
 (segment (start 142.9783 111.785) (end 142.9783 112.3826) (width 0.25) (layer F.Cu) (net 27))
 (segment (start 142.9783 112.3826) (end 153.0491 122.4534) (width 0.25) (layer F.Cu) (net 27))
 (segment (start 153.0491 122.4534) (end 172.4576 122.4534) (width 0.25) (layer F.Cu) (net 27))
 (segment (start 172.4576 122.4534) (end 173.3091 123.3049) (width 0.25) (layer F.Cu) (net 27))
 (segment (start 173.3091 123.3049) (end 173.3091 123.825) (width 0.25) (layer F.Cu) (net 27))
 (segment (start 130.9829 75.565) (end 130.9829 75.0449) (width 0.25) (layer B.Cu) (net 27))
 (segment (start 130.9829 75.0449) (end 131.8136 74.2142) (width 0.25) (layer B.Cu) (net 27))
 (segment (start 131.8136 74.2142) (end 137.9146 74.2142) (width 0.25) (layer B.Cu) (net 27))
 (segment (start 137.9146 74.2142) (end 138.7331 75.0327) (width 0.25) (layer B.Cu) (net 27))
 (segment (start 138.7331 75.0327) (end 138.7331 98.8197) (width 0.25) (layer B.Cu) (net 27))
 (segment (start 138.7331 98.8197) (end 141.783 101.8696) (width 0.25) (layer B.Cu) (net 27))
 (segment (start 141.783 101.8696) (end 141.783 111.785) (width 0.25) (layer B.Cu) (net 27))
 (segment (start 162.7367 102.184) (end 162.7367 87.7183) (width 0.25) (layer B.Cu) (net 23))
 (segment (start 162.7367 87.7183) (end 154.3118 79.2934) (width 0.25) (layer B.Cu) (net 23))
 (segment (start 154.3118 79.2934) (end 154.3118 77.2228) (width 0.25) (layer B.Cu) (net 23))
 (segment (start 154.3118 77.2228) (end 152.654 75.565) (width 0.25) (layer B.Cu) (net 23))
 (segment (start 163.932 102.184) (end 162.7367 102.184) (width 0.25) (layer B.Cu) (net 23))
 (segment (start 156.718 75.565) (end 157.9069 75.565) (width 0.25) (layer F.Cu) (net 17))
 (segment (start 157.9069 75.565) (end 157.9069 75.0449) (width 0.25) (layer F.Cu) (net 17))
 (segment (start 157.9069 75.0449) (end 158.7791 74.1727) (width 0.25) (layer F.Cu) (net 17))
 (segment (start 158.7791 74.1727) (end 159.7629 74.1727) (width 0.25) (layer F.Cu) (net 17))
 (segment (start 159.7629 74.1727) (end 160.528 74.9378) (width 0.25) (layer F.Cu) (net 17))
 (segment (start 160.528 74.9378) (end 160.528 78.8465) (width 0.25) (layer F.Cu) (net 17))
 (segment (start 160.528 78.8465) (end 167.945 86.2635) (width 0.25) (layer F.Cu) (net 17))
 (segment (start 167.945 86.2635) (end 167.945 90.4016) (width 0.25) (layer F.Cu) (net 17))
 (segment (start 167.945 90.4016) (end 173.025 95.4816) (width 0.25) (layer F.Cu) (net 17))
 (segment (start 173.025 95.4816) (end 173.025 112.09) (width 0.25) (layer F.Cu) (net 17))
 (segment (start 161.798 75.565) (end 160.6091 75.565) (width 0.25) (layer B.Cu) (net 8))
 (segment (start 160.6091 75.565) (end 160.6091 76.6011) (width 0.25) (layer B.Cu) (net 8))
 (segment (start 160.6091 76.6011) (end 156.87 80.3402) (width 0.25) (layer B.Cu) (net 8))
 (segment (start 169.215 88.9762) (end 170.4103 88.9762) (width 0.25) (layer B.Cu) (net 21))
 (segment (start 171.958 75.565) (end 170.7691 75.565) (width 0.25) (layer B.Cu) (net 21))
 (segment (start 170.7691 75.565) (end 170.7691 87.4221) (width 0.25) (layer B.Cu) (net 21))
 (segment (start 170.7691 87.4221) (end 170.4103 87.7809) (width 0.25) (layer B.Cu) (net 21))
 (segment (start 170.4103 87.7809) (end 170.4103 88.9762) (width 0.25) (layer B.Cu) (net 21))
 (segment (start 171.755 88.9762) (end 172.9503 88.9762) (width 0.25) (layer B.Cu) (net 20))
 (segment (start 174.498 75.565) (end 174.498 87.4285) (width 0.25) (layer B.Cu) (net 20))
 (segment (start 174.498 87.4285) (end 172.9503 88.9762) (width 0.25) (layer B.Cu) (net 20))
 (segment (start 139.954 75.565) (end 141.1429 75.565) (width 0.25) (layer F.Cu) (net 6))
 (segment (start 141.1429 75.565) (end 141.1429 76.0851) (width 0.25) (layer F.Cu) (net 6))
 (segment (start 141.1429 76.0851) (end 145.398 80.3402) (width 0.25) (layer F.Cu) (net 6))
 (segment (start 145.398 80.3402) (end 151.282 80.3402) (width 0.25) (layer F.Cu) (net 6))
 (segment (start 159.41 80.3402) (end 159.41 81.3655) (width 0.25) (layer F.Cu) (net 9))
 (segment (start 160.274 86.995) (end 160.274 82.2295) (width 0.25) (layer F.Cu) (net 9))
 (segment (start 160.274 82.2295) (end 159.41 81.3655) (width 0.25) (layer F.Cu) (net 9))
 (segment (start 153.822 80.3402) (end 153.822 81.3655) (width 0.25) (layer B.Cu) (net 7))
 (segment (start 154.026 86.995) (end 154.026 81.5695) (width 0.25) (layer B.Cu) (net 7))
 (segment (start 154.026 81.5695) (end 153.822 81.3655) (width 0.25) (layer B.Cu) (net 7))
 (segment (start 128.8582 101.3495) (end 125.832 98.3234) (width 0.25) (layer F.Cu) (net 2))
 (segment (start 134.366 102.286) (end 129.7946 102.286) (width 0.25) (layer F.Cu) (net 2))
 (segment (start 129.7946 102.286) (end 128.8582 101.3495) (width 0.25) (layer F.Cu) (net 2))
 (segment (start 125.832 104.3757) (end 128.8582 101.3495) (width 0.25) (layer F.Cu) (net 2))
 (segment (start 125.832 106.451) (end 125.832 104.3757) (width 0.25) (layer F.Cu) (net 2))
 (segment (start 136.906 102.286) (end 126.7146 112.4774) (width 0.5) (layer F.Cu) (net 4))
 (segment (start 126.7146 112.4774) (end 126.7146 120.3896) (width 0.5) (layer F.Cu) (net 4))
 (segment (start 126.7146 120.3896) (end 130.15 123.825) (width 0.5) (layer F.Cu) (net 4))
 (segment (start 137.2869 101.9051) (end 136.906 102.286) (width 0.5) (layer F.Cu) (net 4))
 (segment (start 163.7944 92.2653) (end 146.9267 92.2653) (width 0.5) (layer F.Cu) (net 4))
 (segment (start 146.9267 92.2653) (end 137.2869 101.9051) (width 0.5) (layer F.Cu) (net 4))
 (segment (start 123.85 88.4682) (end 137.2869 101.9051) (width 0.5) (layer F.Cu) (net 4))
 (segment (start 164.135 88.9762) (end 163.7944 89.3168) (width 0.5) (layer B.Cu) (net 4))
 (segment (start 163.7944 89.3168) (end 163.7944 92.2653) (width 0.5) (layer B.Cu) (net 4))
 (via (at 163.7944 92.2653) (size 0.6) (layers F.Cu B.Cu) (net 4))
 (segment (start 160.1967 102.184) (end 160.1967 100.9887) (width 0.25) (layer B.Cu) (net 24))
 (segment (start 160.1967 100.9887) (end 150.114 90.906) (width 0.25) (layer B.Cu) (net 24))
 (segment (start 150.114 90.906) (end 150.114 76.9063) (width 0.25) (layer B.Cu) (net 24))
 (segment (start 161.392 102.184) (end 160.1967 102.184) (width 0.25) (layer B.Cu) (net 24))
 (segment (start 150.114 75.565) (end 150.114 76.9063) (width 0.25) (layer B.Cu) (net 24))
 (segment (start 157.6567 102.184) (end 157.6567 100.9887) (width 0.25) (layer B.Cu) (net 25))
 (segment (start 157.6567 100.9887) (end 148.5597 91.8917) (width 0.25) (layer B.Cu) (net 25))
 (segment (start 148.5597 91.8917) (end 148.5597 77.892) (width 0.25) (layer B.Cu) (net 25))
 (segment (start 148.5597 77.892) (end 147.574 76.9063) (width 0.25) (layer B.Cu) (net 25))
 (segment (start 158.852 102.184) (end 157.6567 102.184) (width 0.25) (layer B.Cu) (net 25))
 (segment (start 147.574 75.565) (end 147.574 76.9063) (width 0.25) (layer B.Cu) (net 25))
 (segment (start 145.034 75.565) (end 146.2229 75.565) (width 0.25) (layer B.Cu) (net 26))
 (segment (start 146.2229 75.565) (end 146.2229 76.7539) (width 0.25) (layer B.Cu) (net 26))
 (segment (start 146.2229 76.7539) (end 148.1093 78.6403) (width 0.25) (layer B.Cu) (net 26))
 (segment (start 148.1093 78.6403) (end 148.1093 93.9813) (width 0.25) (layer B.Cu) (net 26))
 (segment (start 148.1093 93.9813) (end 156.312 102.184) (width 0.25) (layer B.Cu) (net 26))
 (segment (start 154.381 111.785) (end 155.5763 111.785) (width 0.25) (layer F.Cu) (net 15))
 (segment (start 165.405 112.09) (end 164.2097 112.09) (width 0.25) (layer F.Cu) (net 15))
 (segment (start 164.2097 112.09) (end 164.2097 113.0612) (width 0.25) (layer F.Cu) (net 15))
 (segment (start 164.2097 113.0612) (end 163.739 113.5319) (width 0.25) (layer F.Cu) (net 15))
 (segment (start 163.739 113.5319) (end 156.7255 113.5319) (width 0.25) (layer F.Cu) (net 15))
 (segment (start 156.7255 113.5319) (end 155.5763 112.3827) (width 0.25) (layer F.Cu) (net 15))
 (segment (start 155.5763 112.3827) (end 155.5763 111.785) (width 0.25) (layer F.Cu) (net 15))
 (segment (start 156.921 111.785) (end 155.7257 111.785) (width 0.25) (layer B.Cu) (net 14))
 (segment (start 155.7257 111.785) (end 155.7257 110.5897) (width 0.25) (layer B.Cu) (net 14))
 (segment (start 155.7257 110.5897) (end 141.834 96.698) (width 0.25) (layer B.Cu) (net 14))
 (segment (start 141.834 96.698) (end 141.834 88.5698) (width 0.25) (layer B.Cu) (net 14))
 (segment (start 146.914 88.5698) (end 148.1093 88.5698) (width 0.25) (layer F.Cu) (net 13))
 (segment (start 159.258 75.565) (end 159.258 76.9063) (width 0.25) (layer F.Cu) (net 13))
 (segment (start 159.258 76.9063) (end 158.743 76.9063) (width 0.25) (layer F.Cu) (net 13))
 (segment (start 158.743 76.9063) (end 148.1093 87.54) (width 0.25) (layer F.Cu) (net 13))
 (segment (start 148.1093 87.54) (end 148.1093 88.5698) (width 0.25) (layer F.Cu) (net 13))
 (segment (start 144.374 88.5698) (end 143.1787 88.5698) (width 0.25) (layer F.Cu) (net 11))
 (segment (start 134.01 88.4682) (end 135.2053 88.4682) (width 0.25) (layer F.Cu) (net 11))
 (segment (start 135.2053 88.4682) (end 135.2053 89.0659) (width 0.25) (layer F.Cu) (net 11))
 (segment (start 135.2053 89.0659) (end 136.1427 90.0033) (width 0.25) (layer F.Cu) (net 11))
 (segment (start 136.1427 90.0033) (end 142.7164 90.0033) (width 0.25) (layer F.Cu) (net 11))
 (segment (start 142.7164 90.0033) (end 143.1787 89.541) (width 0.25) (layer F.Cu) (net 11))
 (segment (start 143.1787 89.541) (end 143.1787 88.5698) (width 0.25) (layer F.Cu) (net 11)))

